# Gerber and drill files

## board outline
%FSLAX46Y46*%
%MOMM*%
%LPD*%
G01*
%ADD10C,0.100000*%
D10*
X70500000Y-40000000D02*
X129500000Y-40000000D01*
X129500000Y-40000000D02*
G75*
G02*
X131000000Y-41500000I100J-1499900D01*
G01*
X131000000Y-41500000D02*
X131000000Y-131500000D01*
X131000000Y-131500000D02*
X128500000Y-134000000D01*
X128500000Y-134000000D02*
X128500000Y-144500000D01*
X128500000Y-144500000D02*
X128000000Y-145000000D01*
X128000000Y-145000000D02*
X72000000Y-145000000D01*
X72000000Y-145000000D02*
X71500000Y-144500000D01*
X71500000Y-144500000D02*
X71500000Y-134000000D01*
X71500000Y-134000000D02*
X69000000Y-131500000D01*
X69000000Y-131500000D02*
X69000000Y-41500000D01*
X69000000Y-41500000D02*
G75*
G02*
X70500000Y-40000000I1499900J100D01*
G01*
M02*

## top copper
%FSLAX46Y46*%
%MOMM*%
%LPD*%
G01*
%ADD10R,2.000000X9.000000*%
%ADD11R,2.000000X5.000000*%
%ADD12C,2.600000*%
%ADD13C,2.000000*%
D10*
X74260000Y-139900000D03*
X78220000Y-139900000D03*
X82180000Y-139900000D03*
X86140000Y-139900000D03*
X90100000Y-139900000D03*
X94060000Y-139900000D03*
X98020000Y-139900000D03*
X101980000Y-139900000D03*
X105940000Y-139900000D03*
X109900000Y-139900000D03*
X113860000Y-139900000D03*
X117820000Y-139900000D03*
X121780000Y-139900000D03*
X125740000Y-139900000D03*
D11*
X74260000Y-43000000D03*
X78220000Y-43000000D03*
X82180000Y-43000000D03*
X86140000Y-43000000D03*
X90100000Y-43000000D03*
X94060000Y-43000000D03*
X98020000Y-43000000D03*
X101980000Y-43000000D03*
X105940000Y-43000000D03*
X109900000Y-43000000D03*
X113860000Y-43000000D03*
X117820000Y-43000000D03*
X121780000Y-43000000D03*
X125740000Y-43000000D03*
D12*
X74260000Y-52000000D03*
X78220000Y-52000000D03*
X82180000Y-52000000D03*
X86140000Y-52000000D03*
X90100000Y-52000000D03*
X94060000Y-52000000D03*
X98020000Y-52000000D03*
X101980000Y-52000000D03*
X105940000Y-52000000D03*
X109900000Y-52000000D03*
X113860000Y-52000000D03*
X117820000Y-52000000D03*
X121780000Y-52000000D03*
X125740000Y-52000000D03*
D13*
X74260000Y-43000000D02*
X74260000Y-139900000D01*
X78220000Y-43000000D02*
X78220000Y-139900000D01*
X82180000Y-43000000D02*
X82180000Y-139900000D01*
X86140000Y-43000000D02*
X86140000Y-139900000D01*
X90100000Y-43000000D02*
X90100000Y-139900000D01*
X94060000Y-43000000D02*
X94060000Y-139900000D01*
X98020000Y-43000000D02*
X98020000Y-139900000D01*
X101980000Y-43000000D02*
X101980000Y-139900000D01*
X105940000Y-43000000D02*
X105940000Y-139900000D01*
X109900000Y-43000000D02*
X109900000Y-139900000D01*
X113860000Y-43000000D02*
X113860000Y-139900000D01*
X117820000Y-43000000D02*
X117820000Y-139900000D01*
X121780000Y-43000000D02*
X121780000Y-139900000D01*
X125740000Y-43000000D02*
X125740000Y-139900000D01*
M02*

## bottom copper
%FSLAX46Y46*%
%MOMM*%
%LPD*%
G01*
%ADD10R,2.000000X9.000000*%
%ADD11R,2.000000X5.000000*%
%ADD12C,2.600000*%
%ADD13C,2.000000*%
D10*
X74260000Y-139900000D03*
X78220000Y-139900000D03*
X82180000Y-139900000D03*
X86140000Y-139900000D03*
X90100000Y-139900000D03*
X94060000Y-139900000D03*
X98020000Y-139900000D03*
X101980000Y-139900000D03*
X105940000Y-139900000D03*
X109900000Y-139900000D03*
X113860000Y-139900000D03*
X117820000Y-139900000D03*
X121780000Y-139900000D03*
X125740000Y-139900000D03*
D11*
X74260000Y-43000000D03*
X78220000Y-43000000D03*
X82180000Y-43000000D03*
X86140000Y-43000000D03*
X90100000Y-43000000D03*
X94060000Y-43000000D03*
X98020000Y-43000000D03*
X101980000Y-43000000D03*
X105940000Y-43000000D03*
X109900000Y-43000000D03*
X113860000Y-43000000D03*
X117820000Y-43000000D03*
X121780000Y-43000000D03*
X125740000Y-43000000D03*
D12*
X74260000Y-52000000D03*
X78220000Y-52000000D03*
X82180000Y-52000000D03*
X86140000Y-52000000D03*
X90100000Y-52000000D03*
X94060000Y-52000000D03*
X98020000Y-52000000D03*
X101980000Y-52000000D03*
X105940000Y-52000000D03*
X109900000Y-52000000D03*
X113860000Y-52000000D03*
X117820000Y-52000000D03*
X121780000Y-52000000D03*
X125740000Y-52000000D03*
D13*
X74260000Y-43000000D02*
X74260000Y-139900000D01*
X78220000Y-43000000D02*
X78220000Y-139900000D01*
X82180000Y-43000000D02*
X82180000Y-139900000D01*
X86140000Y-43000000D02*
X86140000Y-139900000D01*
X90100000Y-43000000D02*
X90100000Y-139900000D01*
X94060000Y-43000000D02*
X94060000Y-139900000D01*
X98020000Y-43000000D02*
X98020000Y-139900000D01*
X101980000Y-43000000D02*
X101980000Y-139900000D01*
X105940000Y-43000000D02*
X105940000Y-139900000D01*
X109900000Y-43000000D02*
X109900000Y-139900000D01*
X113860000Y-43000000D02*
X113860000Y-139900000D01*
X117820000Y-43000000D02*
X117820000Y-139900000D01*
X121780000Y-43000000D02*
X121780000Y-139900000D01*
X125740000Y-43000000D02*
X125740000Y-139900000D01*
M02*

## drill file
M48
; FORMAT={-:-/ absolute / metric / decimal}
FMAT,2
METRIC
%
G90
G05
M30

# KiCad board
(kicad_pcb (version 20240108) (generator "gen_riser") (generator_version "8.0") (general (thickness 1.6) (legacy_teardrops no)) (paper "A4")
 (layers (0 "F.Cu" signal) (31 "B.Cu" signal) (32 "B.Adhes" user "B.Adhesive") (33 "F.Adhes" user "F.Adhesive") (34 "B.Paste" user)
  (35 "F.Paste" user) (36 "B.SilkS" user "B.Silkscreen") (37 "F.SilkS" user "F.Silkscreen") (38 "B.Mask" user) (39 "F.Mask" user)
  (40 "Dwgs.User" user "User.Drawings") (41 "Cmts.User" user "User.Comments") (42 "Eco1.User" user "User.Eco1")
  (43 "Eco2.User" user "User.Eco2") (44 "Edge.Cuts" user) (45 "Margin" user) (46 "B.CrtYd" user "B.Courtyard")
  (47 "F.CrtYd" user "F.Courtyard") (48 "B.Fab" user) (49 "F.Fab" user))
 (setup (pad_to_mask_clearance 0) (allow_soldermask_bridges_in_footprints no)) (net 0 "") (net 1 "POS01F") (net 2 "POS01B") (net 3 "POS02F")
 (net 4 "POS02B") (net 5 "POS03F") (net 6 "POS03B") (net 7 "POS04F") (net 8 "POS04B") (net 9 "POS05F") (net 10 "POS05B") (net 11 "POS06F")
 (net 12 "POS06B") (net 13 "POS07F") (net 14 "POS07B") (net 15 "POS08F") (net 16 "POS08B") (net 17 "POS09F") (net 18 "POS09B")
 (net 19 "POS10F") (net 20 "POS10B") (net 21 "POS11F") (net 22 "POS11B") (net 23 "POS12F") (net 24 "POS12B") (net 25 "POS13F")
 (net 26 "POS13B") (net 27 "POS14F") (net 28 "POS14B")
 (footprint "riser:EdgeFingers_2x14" (layer "F.Cu") (at 100 40)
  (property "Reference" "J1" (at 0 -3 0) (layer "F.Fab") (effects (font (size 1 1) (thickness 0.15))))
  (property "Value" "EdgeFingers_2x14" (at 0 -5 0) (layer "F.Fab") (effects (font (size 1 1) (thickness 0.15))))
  (pad "1" smd rect (at -25.74 99.9) (size 2 9) (layers "F.Cu" "F.Mask") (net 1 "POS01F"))
  (pad "1B" smd rect (at -25.74 99.9) (size 2 9) (layers "B.Cu" "B.Mask") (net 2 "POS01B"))
  (pad "2" smd rect (at -21.78 99.9) (size 2 9) (layers "F.Cu" "F.Mask") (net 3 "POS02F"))
  (pad "2B" smd rect (at -21.78 99.9) (size 2 9) (layers "B.Cu" "B.Mask") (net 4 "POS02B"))
  (pad "3" smd rect (at -17.82 99.9) (size 2 9) (layers "F.Cu" "F.Mask") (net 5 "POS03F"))
  (pad "3B" smd rect (at -17.82 99.9) (size 2 9) (layers "B.Cu" "B.Mask") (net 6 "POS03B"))
  (pad "4" smd rect (at -13.86 99.9) (size 2 9) (layers "F.Cu" "F.Mask") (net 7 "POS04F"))
  (pad "4B" smd rect (at -13.86 99.9) (size 2 9) (layers "B.Cu" "B.Mask") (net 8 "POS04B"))
  (pad "5" smd rect (at -9.9 99.9) (size 2 9) (layers "F.Cu" "F.Mask") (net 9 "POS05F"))
  (pad "5B" smd rect (at -9.9 99.9) (size 2 9) (layers "B.Cu" "B.Mask") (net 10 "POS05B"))
  (pad "6" smd rect (at -5.94 99.9) (size 2 9) (layers "F.Cu" "F.Mask") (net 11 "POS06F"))
  (pad "6B" smd rect (at -5.94 99.9) (size 2 9) (layers "B.Cu" "B.Mask") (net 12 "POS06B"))
  (pad "7" smd rect (at -1.98 99.9) (size 2 9) (layers "F.Cu" "F.Mask") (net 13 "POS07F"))
  (pad "7B" smd rect (at -1.98 99.9) (size 2 9) (layers "B.Cu" "B.Mask") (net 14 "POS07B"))
  (pad "8" smd rect (at 1.98 99.9) (size 2 9) (layers "F.Cu" "F.Mask") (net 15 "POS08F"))
  (pad "8B" smd rect (at 1.98 99.9) (size 2 9) (layers "B.Cu" "B.Mask") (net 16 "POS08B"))
  (pad "9" smd rect (at 5.94 99.9) (size 2 9) (layers "F.Cu" "F.Mask") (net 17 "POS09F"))
  (pad "9B" smd rect (at 5.94 99.9) (size 2 9) (layers "B.Cu" "B.Mask") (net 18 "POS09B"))
  (pad "10" smd rect (at 9.9 99.9) (size 2 9) (layers "F.Cu" "F.Mask") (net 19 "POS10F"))
  (pad "10B" smd rect (at 9.9 99.9) (size 2 9) (layers "B.Cu" "B.Mask") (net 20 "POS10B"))
  (pad "11" smd rect (at 13.86 99.9) (size 2 9) (layers "F.Cu" "F.Mask") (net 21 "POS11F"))
  (pad "11B" smd rect (at 13.86 99.9) (size 2 9) (layers "B.Cu" "B.Mask") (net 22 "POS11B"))
  (pad "12" smd rect (at 17.82 99.9) (size 2 9) (layers "F.Cu" "F.Mask") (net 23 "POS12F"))
  (pad "12B" smd rect (at 17.82 99.9) (size 2 9) (layers "B.Cu" "B.Mask") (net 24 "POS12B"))
  (pad "13" smd rect (at 21.78 99.9) (size 2 9) (layers "F.Cu" "F.Mask") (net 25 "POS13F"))
  (pad "13B" smd rect (at 21.78 99.9) (size 2 9) (layers "B.Cu" "B.Mask") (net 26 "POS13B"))
  (pad "14" smd rect (at 25.74 99.9) (size 2 9) (layers "F.Cu" "F.Mask") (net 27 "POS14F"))
  (pad "14B" smd rect (at 25.74 99.9) (size 2 9) (layers "B.Cu" "B.Mask") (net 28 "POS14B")))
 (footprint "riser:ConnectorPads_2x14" (layer "F.Cu") (at 100 40)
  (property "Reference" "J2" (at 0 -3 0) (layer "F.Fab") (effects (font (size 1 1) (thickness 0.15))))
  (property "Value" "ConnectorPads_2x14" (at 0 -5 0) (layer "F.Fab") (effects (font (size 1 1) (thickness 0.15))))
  (pad "1" smd rect (at -25.74 3) (size 2 5) (layers "F.Cu" "F.Mask") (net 1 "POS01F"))
  (pad "1B" smd rect (at -25.74 3) (size 2 5) (layers "B.Cu" "B.Mask") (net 2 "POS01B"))
  (pad "2" smd rect (at -21.78 3) (size 2 5) (layers "F.Cu" "F.Mask") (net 3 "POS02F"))
  (pad "2B" smd rect (at -21.78 3) (size 2 5) (layers "B.Cu" "B.Mask") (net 4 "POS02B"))
  (pad "3" smd rect (at -17.82 3) (size 2 5) (layers "F.Cu" "F.Mask") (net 5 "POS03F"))
  (pad "3B" smd rect (at -17.82 3) (size 2 5) (layers "B.Cu" "B.Mask") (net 6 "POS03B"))
  (pad "4" smd rect (at -13.86 3) (size 2 5) (layers "F.Cu" "F.Mask") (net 7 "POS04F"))
  (pad "4B" smd rect (at -13.86 3) (size 2 5) (layers "B.Cu" "B.Mask") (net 8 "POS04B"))
  (pad "5" smd rect (at -9.9 3) (size 2 5) (layers "F.Cu" "F.Mask") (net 9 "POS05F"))
  (pad "5B" smd rect (at -9.9 3) (size 2 5) (layers "B.Cu" "B.Mask") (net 10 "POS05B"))
  (pad "6" smd rect (at -5.94 3) (size 2 5) (layers "F.Cu" "F.Mask") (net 11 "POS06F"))
  (pad "6B" smd rect (at -5.94 3) (size 2 5) (layers "B.Cu" "B.Mask") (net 12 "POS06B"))
  (pad "7" smd rect (at -1.98 3) (size 2 5) (layers "F.Cu" "F.Mask") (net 13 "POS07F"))
  (pad "7B" smd rect (at -1.98 3) (size 2 5) (layers "B.Cu" "B.Mask") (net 14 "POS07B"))
  (pad "8" smd rect (at 1.98 3) (size 2 5) (layers "F.Cu" "F.Mask") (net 15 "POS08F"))
  (pad "8B" smd rect (at 1.98 3) (size 2 5) (layers "B.Cu" "B.Mask") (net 16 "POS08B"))
  (pad "9" smd rect (at 5.94 3) (size 2 5) (layers "F.Cu" "F.Mask") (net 17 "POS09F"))
  (pad "9B" smd rect (at 5.94 3) (size 2 5) (layers "B.Cu" "B.Mask") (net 18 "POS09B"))
  (pad "10" smd rect (at 9.9 3) (size 2 5) (layers "F.Cu" "F.Mask") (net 19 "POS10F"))
  (pad "10B" smd rect (at 9.9 3) (size 2 5) (layers "B.Cu" "B.Mask") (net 20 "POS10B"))
  (pad "11" smd rect (at 13.86 3) (size 2 5) (layers "F.Cu" "F.Mask") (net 21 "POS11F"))
  (pad "11B" smd rect (at 13.86 3) (size 2 5) (layers "B.Cu" "B.Mask") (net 22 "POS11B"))
  (pad "12" smd rect (at 17.82 3) (size 2 5) (layers "F.Cu" "F.Mask") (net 23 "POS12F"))
  (pad "12B" smd rect (at 17.82 3) (size 2 5) (layers "B.Cu" "B.Mask") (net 24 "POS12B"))
  (pad "13" smd rect (at 21.78 3) (size 2 5) (layers "F.Cu" "F.Mask") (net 25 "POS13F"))
  (pad "13B" smd rect (at 21.78 3) (size 2 5) (layers "B.Cu" "B.Mask") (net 26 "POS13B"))
  (pad "14" smd rect (at 25.74 3) (size 2 5) (layers "F.Cu" "F.Mask") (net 27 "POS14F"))
  (pad "14B" smd rect (at 25.74 3) (size 2 5) (layers "B.Cu" "B.Mask") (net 28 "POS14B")))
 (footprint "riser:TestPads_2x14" (layer "F.Cu") (at 100 40)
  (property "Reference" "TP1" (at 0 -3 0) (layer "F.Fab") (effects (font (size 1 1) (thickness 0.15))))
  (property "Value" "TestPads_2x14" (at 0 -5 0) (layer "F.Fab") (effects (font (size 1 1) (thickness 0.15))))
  (pad "1" smd circle (at -25.74 12) (size 2.6 2.6) (layers "F.Cu" "F.Mask") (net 1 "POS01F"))
  (pad "1B" smd circle (at -25.74 12) (size 2.6 2.6) (layers "B.Cu" "B.Mask") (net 2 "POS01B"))
  (pad "2" smd circle (at -21.78 12) (size 2.6 2.6) (layers "F.Cu" "F.Mask") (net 3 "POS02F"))
  (pad "2B" smd circle (at -21.78 12) (size 2.6 2.6) (layers "B.Cu" "B.Mask") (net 4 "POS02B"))
  (pad "3" smd circle (at -17.82 12) (size 2.6 2.6) (layers "F.Cu" "F.Mask") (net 5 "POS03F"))
  (pad "3B" smd circle (at -17.82 12) (size 2.6 2.6) (layers "B.Cu" "B.Mask") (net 6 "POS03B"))
  (pad "4" smd circle (at -13.86 12) (size 2.6 2.6) (layers "F.Cu" "F.Mask") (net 7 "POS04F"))
  (pad "4B" smd circle (at -13.86 12) (size 2.6 2.6) (layers "B.Cu" "B.Mask") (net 8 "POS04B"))
  (pad "5" smd circle (at -9.9 12) (size 2.6 2.6) (layers "F.Cu" "F.Mask") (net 9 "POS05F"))
  (pad "5B" smd circle (at -9.9 12) (size 2.6 2.6) (layers "B.Cu" "B.Mask") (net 10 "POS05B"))
  (pad "6" smd circle (at -5.94 12) (size 2.6 2.6) (layers "F.Cu" "F.Mask") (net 11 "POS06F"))
  (pad "6B" smd circle (at -5.94 12) (size 2.6 2.6) (layers "B.Cu" "B.Mask") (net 12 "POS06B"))
  (pad "7" smd circle (at -1.98 12) (size 2.6 2.6) (layers "F.Cu" "F.Mask") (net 13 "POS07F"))
  (pad "7B" smd circle (at -1.98 12) (size 2.6 2.6) (layers "B.Cu" "B.Mask") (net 14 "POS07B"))
  (pad "8" smd circle (at 1.98 12) (size 2.6 2.6) (layers "F.Cu" "F.Mask") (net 15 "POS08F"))
  (pad "8B" smd circle (at 1.98 12) (size 2.6 2.6) (layers "B.Cu" "B.Mask") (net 16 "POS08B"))
  (pad "9" smd circle (at 5.94 12) (size 2.6 2.6) (layers "F.Cu" "F.Mask") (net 17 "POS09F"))
  (pad "9B" smd circle (at 5.94 12) (size 2.6 2.6) (layers "B.Cu" "B.Mask") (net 18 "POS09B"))
  (pad "10" smd circle (at 9.9 12) (size 2.6 2.6) (layers "F.Cu" "F.Mask") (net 19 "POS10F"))
  (pad "10B" smd circle (at 9.9 12) (size 2.6 2.6) (layers "B.Cu" "B.Mask") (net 20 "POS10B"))
  (pad "11" smd circle (at 13.86 12) (size 2.6 2.6) (layers "F.Cu" "F.Mask") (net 21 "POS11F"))
  (pad "11B" smd circle (at 13.86 12) (size 2.6 2.6) (layers "B.Cu" "B.Mask") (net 22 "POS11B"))
  (pad "12" smd circle (at 17.82 12) (size 2.6 2.6) (layers "F.Cu" "F.Mask") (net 23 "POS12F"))
  (pad "12B" smd circle (at 17.82 12) (size 2.6 2.6) (layers "B.Cu" "B.Mask") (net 24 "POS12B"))
  (pad "13" smd circle (at 21.78 12) (size 2.6 2.6) (layers "F.Cu" "F.Mask") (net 25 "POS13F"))
  (pad "13B" smd circle (at 21.78 12) (size 2.6 2.6) (layers "B.Cu" "B.Mask") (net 26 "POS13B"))
  (pad "14" smd circle (at 25.74 12) (size 2.6 2.6) (layers "F.Cu" "F.Mask") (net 27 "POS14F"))
  (pad "14B" smd circle (at 25.74 12) (size 2.6 2.6) (layers "B.Cu" "B.Mask") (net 28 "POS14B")))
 (segment (start 74.26 43) (end 74.26 139.9) (width 2) (layer "F.Cu") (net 1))
 (segment (start 74.26 43) (end 74.26 139.9) (width 2) (layer "B.Cu") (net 2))
 (segment (start 78.22 43) (end 78.22 139.9) (width 2) (layer "F.Cu") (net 3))
 (segment (start 78.22 43) (end 78.22 139.9) (width 2) (layer "B.Cu") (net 4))
 (segment (start 82.18 43) (end 82.18 139.9) (width 2) (layer "F.Cu") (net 5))
 (segment (start 82.18 43) (end 82.18 139.9) (width 2) (layer "B.Cu") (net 6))
 (segment (start 86.14 43) (end 86.14 139.9) (width 2) (layer "F.Cu") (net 7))
 (segment (start 86.14 43) (end 86.14 139.9) (width 2) (layer "B.Cu") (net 8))
 (segment (start 90.1 43) (end 90.1 139.9) (width 2) (layer "F.Cu") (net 9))
 (segment (start 90.1 43) (end 90.1 139.9) (width 2) (layer "B.Cu") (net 10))
 (segment (start 94.06 43) (end 94.06 139.9) (width 2) (layer "F.Cu") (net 11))
 (segment (start 94.06 43) (end 94.06 139.9) (width 2) (layer "B.Cu") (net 12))
 (segment (start 98.02 43) (end 98.02 139.9) (width 2) (layer "F.Cu") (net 13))
 (segment (start 98.02 43) (end 98.02 139.9) (width 2) (layer "B.Cu") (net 14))
 (segment (start 101.98 43) (end 101.98 139.9) (width 2) (layer "F.Cu") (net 15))
 (segment (start 101.98 43) (end 101.98 139.9) (width 2) (layer "B.Cu") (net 16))
 (segment (start 105.94 43) (end 105.94 139.9) (width 2) (layer "F.Cu") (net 17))
 (segment (start 105.94 43) (end 105.94 139.9) (width 2) (layer "B.Cu") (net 18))
 (segment (start 109.9 43) (end 109.9 139.9) (width 2) (layer "F.Cu") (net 19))
 (segment (start 109.9 43) (end 109.9 139.9) (width 2) (layer "B.Cu") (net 20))
 (segment (start 113.86 43) (end 113.86 139.9) (width 2) (layer "F.Cu") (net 21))
 (segment (start 113.86 43) (end 113.86 139.9) (width 2) (layer "B.Cu") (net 22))
 (segment (start 117.82 43) (end 117.82 139.9) (width 2) (layer "F.Cu") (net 23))
 (segment (start 117.82 43) (end 117.82 139.9) (width 2) (layer "B.Cu") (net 24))
 (segment (start 121.78 43) (end 121.78 139.9) (width 2) (layer "F.Cu") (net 25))
 (segment (start 121.78 43) (end 121.78 139.9) (width 2) (layer "B.Cu") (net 26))
 (segment (start 125.74 43) (end 125.74 139.9) (width 2) (layer "F.Cu") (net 27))
 (segment (start 125.74 43) (end 125.74 139.9) (width 2) (layer "B.Cu") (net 28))
 (gr_line (start 70.5 40) (end 129.5 40) (stroke (width 0.1) (type default)) (layer "Edge.Cuts"))
 (gr_arc (start 129.5 40) (mid 130.5607 40.4393) (end 131 41.5) (stroke (width 0.1) (type default)) (layer "Edge.Cuts"))
 (gr_line (start 131 41.5) (end 131 131.5) (stroke (width 0.1) (type default)) (layer "Edge.Cuts"))
 (gr_line (start 131 131.5) (end 128.5 134) (stroke (width 0.1) (type default)) (layer "Edge.Cuts"))
 (gr_line (start 128.5 134) (end 128.5 144.5) (stroke (width 0.1) (type default)) (layer "Edge.Cuts"))
 (gr_line (start 128.5 144.5) (end 128 145) (stroke (width 0.1) (type default)) (layer "Edge.Cuts"))
 (gr_line (start 128 145) (end 72 145) (stroke (width 0.1) (type default)) (layer "Edge.Cuts"))
 (gr_line (start 72 145) (end 71.5 144.5) (stroke (width 0.1) (type default)) (layer "Edge.Cuts"))
 (gr_line (start 71.5 144.5) (end 71.5 134) (stroke (width 0.1) (type default)) (layer "Edge.Cuts"))
 (gr_line (start 71.5 134) (end 69 131.5) (stroke (width 0.1) (type default)) (layer "Edge.Cuts"))
 (gr_line (start 69 131.5) (end 69 41.5) (stroke (width 0.1) (type default)) (layer "Edge.Cuts"))
 (gr_arc (start 69 41.5) (mid 69.4393 40.4393) (end 70.5 40) (stroke (width 0.1) (type default)) (layer "Edge.Cuts")))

